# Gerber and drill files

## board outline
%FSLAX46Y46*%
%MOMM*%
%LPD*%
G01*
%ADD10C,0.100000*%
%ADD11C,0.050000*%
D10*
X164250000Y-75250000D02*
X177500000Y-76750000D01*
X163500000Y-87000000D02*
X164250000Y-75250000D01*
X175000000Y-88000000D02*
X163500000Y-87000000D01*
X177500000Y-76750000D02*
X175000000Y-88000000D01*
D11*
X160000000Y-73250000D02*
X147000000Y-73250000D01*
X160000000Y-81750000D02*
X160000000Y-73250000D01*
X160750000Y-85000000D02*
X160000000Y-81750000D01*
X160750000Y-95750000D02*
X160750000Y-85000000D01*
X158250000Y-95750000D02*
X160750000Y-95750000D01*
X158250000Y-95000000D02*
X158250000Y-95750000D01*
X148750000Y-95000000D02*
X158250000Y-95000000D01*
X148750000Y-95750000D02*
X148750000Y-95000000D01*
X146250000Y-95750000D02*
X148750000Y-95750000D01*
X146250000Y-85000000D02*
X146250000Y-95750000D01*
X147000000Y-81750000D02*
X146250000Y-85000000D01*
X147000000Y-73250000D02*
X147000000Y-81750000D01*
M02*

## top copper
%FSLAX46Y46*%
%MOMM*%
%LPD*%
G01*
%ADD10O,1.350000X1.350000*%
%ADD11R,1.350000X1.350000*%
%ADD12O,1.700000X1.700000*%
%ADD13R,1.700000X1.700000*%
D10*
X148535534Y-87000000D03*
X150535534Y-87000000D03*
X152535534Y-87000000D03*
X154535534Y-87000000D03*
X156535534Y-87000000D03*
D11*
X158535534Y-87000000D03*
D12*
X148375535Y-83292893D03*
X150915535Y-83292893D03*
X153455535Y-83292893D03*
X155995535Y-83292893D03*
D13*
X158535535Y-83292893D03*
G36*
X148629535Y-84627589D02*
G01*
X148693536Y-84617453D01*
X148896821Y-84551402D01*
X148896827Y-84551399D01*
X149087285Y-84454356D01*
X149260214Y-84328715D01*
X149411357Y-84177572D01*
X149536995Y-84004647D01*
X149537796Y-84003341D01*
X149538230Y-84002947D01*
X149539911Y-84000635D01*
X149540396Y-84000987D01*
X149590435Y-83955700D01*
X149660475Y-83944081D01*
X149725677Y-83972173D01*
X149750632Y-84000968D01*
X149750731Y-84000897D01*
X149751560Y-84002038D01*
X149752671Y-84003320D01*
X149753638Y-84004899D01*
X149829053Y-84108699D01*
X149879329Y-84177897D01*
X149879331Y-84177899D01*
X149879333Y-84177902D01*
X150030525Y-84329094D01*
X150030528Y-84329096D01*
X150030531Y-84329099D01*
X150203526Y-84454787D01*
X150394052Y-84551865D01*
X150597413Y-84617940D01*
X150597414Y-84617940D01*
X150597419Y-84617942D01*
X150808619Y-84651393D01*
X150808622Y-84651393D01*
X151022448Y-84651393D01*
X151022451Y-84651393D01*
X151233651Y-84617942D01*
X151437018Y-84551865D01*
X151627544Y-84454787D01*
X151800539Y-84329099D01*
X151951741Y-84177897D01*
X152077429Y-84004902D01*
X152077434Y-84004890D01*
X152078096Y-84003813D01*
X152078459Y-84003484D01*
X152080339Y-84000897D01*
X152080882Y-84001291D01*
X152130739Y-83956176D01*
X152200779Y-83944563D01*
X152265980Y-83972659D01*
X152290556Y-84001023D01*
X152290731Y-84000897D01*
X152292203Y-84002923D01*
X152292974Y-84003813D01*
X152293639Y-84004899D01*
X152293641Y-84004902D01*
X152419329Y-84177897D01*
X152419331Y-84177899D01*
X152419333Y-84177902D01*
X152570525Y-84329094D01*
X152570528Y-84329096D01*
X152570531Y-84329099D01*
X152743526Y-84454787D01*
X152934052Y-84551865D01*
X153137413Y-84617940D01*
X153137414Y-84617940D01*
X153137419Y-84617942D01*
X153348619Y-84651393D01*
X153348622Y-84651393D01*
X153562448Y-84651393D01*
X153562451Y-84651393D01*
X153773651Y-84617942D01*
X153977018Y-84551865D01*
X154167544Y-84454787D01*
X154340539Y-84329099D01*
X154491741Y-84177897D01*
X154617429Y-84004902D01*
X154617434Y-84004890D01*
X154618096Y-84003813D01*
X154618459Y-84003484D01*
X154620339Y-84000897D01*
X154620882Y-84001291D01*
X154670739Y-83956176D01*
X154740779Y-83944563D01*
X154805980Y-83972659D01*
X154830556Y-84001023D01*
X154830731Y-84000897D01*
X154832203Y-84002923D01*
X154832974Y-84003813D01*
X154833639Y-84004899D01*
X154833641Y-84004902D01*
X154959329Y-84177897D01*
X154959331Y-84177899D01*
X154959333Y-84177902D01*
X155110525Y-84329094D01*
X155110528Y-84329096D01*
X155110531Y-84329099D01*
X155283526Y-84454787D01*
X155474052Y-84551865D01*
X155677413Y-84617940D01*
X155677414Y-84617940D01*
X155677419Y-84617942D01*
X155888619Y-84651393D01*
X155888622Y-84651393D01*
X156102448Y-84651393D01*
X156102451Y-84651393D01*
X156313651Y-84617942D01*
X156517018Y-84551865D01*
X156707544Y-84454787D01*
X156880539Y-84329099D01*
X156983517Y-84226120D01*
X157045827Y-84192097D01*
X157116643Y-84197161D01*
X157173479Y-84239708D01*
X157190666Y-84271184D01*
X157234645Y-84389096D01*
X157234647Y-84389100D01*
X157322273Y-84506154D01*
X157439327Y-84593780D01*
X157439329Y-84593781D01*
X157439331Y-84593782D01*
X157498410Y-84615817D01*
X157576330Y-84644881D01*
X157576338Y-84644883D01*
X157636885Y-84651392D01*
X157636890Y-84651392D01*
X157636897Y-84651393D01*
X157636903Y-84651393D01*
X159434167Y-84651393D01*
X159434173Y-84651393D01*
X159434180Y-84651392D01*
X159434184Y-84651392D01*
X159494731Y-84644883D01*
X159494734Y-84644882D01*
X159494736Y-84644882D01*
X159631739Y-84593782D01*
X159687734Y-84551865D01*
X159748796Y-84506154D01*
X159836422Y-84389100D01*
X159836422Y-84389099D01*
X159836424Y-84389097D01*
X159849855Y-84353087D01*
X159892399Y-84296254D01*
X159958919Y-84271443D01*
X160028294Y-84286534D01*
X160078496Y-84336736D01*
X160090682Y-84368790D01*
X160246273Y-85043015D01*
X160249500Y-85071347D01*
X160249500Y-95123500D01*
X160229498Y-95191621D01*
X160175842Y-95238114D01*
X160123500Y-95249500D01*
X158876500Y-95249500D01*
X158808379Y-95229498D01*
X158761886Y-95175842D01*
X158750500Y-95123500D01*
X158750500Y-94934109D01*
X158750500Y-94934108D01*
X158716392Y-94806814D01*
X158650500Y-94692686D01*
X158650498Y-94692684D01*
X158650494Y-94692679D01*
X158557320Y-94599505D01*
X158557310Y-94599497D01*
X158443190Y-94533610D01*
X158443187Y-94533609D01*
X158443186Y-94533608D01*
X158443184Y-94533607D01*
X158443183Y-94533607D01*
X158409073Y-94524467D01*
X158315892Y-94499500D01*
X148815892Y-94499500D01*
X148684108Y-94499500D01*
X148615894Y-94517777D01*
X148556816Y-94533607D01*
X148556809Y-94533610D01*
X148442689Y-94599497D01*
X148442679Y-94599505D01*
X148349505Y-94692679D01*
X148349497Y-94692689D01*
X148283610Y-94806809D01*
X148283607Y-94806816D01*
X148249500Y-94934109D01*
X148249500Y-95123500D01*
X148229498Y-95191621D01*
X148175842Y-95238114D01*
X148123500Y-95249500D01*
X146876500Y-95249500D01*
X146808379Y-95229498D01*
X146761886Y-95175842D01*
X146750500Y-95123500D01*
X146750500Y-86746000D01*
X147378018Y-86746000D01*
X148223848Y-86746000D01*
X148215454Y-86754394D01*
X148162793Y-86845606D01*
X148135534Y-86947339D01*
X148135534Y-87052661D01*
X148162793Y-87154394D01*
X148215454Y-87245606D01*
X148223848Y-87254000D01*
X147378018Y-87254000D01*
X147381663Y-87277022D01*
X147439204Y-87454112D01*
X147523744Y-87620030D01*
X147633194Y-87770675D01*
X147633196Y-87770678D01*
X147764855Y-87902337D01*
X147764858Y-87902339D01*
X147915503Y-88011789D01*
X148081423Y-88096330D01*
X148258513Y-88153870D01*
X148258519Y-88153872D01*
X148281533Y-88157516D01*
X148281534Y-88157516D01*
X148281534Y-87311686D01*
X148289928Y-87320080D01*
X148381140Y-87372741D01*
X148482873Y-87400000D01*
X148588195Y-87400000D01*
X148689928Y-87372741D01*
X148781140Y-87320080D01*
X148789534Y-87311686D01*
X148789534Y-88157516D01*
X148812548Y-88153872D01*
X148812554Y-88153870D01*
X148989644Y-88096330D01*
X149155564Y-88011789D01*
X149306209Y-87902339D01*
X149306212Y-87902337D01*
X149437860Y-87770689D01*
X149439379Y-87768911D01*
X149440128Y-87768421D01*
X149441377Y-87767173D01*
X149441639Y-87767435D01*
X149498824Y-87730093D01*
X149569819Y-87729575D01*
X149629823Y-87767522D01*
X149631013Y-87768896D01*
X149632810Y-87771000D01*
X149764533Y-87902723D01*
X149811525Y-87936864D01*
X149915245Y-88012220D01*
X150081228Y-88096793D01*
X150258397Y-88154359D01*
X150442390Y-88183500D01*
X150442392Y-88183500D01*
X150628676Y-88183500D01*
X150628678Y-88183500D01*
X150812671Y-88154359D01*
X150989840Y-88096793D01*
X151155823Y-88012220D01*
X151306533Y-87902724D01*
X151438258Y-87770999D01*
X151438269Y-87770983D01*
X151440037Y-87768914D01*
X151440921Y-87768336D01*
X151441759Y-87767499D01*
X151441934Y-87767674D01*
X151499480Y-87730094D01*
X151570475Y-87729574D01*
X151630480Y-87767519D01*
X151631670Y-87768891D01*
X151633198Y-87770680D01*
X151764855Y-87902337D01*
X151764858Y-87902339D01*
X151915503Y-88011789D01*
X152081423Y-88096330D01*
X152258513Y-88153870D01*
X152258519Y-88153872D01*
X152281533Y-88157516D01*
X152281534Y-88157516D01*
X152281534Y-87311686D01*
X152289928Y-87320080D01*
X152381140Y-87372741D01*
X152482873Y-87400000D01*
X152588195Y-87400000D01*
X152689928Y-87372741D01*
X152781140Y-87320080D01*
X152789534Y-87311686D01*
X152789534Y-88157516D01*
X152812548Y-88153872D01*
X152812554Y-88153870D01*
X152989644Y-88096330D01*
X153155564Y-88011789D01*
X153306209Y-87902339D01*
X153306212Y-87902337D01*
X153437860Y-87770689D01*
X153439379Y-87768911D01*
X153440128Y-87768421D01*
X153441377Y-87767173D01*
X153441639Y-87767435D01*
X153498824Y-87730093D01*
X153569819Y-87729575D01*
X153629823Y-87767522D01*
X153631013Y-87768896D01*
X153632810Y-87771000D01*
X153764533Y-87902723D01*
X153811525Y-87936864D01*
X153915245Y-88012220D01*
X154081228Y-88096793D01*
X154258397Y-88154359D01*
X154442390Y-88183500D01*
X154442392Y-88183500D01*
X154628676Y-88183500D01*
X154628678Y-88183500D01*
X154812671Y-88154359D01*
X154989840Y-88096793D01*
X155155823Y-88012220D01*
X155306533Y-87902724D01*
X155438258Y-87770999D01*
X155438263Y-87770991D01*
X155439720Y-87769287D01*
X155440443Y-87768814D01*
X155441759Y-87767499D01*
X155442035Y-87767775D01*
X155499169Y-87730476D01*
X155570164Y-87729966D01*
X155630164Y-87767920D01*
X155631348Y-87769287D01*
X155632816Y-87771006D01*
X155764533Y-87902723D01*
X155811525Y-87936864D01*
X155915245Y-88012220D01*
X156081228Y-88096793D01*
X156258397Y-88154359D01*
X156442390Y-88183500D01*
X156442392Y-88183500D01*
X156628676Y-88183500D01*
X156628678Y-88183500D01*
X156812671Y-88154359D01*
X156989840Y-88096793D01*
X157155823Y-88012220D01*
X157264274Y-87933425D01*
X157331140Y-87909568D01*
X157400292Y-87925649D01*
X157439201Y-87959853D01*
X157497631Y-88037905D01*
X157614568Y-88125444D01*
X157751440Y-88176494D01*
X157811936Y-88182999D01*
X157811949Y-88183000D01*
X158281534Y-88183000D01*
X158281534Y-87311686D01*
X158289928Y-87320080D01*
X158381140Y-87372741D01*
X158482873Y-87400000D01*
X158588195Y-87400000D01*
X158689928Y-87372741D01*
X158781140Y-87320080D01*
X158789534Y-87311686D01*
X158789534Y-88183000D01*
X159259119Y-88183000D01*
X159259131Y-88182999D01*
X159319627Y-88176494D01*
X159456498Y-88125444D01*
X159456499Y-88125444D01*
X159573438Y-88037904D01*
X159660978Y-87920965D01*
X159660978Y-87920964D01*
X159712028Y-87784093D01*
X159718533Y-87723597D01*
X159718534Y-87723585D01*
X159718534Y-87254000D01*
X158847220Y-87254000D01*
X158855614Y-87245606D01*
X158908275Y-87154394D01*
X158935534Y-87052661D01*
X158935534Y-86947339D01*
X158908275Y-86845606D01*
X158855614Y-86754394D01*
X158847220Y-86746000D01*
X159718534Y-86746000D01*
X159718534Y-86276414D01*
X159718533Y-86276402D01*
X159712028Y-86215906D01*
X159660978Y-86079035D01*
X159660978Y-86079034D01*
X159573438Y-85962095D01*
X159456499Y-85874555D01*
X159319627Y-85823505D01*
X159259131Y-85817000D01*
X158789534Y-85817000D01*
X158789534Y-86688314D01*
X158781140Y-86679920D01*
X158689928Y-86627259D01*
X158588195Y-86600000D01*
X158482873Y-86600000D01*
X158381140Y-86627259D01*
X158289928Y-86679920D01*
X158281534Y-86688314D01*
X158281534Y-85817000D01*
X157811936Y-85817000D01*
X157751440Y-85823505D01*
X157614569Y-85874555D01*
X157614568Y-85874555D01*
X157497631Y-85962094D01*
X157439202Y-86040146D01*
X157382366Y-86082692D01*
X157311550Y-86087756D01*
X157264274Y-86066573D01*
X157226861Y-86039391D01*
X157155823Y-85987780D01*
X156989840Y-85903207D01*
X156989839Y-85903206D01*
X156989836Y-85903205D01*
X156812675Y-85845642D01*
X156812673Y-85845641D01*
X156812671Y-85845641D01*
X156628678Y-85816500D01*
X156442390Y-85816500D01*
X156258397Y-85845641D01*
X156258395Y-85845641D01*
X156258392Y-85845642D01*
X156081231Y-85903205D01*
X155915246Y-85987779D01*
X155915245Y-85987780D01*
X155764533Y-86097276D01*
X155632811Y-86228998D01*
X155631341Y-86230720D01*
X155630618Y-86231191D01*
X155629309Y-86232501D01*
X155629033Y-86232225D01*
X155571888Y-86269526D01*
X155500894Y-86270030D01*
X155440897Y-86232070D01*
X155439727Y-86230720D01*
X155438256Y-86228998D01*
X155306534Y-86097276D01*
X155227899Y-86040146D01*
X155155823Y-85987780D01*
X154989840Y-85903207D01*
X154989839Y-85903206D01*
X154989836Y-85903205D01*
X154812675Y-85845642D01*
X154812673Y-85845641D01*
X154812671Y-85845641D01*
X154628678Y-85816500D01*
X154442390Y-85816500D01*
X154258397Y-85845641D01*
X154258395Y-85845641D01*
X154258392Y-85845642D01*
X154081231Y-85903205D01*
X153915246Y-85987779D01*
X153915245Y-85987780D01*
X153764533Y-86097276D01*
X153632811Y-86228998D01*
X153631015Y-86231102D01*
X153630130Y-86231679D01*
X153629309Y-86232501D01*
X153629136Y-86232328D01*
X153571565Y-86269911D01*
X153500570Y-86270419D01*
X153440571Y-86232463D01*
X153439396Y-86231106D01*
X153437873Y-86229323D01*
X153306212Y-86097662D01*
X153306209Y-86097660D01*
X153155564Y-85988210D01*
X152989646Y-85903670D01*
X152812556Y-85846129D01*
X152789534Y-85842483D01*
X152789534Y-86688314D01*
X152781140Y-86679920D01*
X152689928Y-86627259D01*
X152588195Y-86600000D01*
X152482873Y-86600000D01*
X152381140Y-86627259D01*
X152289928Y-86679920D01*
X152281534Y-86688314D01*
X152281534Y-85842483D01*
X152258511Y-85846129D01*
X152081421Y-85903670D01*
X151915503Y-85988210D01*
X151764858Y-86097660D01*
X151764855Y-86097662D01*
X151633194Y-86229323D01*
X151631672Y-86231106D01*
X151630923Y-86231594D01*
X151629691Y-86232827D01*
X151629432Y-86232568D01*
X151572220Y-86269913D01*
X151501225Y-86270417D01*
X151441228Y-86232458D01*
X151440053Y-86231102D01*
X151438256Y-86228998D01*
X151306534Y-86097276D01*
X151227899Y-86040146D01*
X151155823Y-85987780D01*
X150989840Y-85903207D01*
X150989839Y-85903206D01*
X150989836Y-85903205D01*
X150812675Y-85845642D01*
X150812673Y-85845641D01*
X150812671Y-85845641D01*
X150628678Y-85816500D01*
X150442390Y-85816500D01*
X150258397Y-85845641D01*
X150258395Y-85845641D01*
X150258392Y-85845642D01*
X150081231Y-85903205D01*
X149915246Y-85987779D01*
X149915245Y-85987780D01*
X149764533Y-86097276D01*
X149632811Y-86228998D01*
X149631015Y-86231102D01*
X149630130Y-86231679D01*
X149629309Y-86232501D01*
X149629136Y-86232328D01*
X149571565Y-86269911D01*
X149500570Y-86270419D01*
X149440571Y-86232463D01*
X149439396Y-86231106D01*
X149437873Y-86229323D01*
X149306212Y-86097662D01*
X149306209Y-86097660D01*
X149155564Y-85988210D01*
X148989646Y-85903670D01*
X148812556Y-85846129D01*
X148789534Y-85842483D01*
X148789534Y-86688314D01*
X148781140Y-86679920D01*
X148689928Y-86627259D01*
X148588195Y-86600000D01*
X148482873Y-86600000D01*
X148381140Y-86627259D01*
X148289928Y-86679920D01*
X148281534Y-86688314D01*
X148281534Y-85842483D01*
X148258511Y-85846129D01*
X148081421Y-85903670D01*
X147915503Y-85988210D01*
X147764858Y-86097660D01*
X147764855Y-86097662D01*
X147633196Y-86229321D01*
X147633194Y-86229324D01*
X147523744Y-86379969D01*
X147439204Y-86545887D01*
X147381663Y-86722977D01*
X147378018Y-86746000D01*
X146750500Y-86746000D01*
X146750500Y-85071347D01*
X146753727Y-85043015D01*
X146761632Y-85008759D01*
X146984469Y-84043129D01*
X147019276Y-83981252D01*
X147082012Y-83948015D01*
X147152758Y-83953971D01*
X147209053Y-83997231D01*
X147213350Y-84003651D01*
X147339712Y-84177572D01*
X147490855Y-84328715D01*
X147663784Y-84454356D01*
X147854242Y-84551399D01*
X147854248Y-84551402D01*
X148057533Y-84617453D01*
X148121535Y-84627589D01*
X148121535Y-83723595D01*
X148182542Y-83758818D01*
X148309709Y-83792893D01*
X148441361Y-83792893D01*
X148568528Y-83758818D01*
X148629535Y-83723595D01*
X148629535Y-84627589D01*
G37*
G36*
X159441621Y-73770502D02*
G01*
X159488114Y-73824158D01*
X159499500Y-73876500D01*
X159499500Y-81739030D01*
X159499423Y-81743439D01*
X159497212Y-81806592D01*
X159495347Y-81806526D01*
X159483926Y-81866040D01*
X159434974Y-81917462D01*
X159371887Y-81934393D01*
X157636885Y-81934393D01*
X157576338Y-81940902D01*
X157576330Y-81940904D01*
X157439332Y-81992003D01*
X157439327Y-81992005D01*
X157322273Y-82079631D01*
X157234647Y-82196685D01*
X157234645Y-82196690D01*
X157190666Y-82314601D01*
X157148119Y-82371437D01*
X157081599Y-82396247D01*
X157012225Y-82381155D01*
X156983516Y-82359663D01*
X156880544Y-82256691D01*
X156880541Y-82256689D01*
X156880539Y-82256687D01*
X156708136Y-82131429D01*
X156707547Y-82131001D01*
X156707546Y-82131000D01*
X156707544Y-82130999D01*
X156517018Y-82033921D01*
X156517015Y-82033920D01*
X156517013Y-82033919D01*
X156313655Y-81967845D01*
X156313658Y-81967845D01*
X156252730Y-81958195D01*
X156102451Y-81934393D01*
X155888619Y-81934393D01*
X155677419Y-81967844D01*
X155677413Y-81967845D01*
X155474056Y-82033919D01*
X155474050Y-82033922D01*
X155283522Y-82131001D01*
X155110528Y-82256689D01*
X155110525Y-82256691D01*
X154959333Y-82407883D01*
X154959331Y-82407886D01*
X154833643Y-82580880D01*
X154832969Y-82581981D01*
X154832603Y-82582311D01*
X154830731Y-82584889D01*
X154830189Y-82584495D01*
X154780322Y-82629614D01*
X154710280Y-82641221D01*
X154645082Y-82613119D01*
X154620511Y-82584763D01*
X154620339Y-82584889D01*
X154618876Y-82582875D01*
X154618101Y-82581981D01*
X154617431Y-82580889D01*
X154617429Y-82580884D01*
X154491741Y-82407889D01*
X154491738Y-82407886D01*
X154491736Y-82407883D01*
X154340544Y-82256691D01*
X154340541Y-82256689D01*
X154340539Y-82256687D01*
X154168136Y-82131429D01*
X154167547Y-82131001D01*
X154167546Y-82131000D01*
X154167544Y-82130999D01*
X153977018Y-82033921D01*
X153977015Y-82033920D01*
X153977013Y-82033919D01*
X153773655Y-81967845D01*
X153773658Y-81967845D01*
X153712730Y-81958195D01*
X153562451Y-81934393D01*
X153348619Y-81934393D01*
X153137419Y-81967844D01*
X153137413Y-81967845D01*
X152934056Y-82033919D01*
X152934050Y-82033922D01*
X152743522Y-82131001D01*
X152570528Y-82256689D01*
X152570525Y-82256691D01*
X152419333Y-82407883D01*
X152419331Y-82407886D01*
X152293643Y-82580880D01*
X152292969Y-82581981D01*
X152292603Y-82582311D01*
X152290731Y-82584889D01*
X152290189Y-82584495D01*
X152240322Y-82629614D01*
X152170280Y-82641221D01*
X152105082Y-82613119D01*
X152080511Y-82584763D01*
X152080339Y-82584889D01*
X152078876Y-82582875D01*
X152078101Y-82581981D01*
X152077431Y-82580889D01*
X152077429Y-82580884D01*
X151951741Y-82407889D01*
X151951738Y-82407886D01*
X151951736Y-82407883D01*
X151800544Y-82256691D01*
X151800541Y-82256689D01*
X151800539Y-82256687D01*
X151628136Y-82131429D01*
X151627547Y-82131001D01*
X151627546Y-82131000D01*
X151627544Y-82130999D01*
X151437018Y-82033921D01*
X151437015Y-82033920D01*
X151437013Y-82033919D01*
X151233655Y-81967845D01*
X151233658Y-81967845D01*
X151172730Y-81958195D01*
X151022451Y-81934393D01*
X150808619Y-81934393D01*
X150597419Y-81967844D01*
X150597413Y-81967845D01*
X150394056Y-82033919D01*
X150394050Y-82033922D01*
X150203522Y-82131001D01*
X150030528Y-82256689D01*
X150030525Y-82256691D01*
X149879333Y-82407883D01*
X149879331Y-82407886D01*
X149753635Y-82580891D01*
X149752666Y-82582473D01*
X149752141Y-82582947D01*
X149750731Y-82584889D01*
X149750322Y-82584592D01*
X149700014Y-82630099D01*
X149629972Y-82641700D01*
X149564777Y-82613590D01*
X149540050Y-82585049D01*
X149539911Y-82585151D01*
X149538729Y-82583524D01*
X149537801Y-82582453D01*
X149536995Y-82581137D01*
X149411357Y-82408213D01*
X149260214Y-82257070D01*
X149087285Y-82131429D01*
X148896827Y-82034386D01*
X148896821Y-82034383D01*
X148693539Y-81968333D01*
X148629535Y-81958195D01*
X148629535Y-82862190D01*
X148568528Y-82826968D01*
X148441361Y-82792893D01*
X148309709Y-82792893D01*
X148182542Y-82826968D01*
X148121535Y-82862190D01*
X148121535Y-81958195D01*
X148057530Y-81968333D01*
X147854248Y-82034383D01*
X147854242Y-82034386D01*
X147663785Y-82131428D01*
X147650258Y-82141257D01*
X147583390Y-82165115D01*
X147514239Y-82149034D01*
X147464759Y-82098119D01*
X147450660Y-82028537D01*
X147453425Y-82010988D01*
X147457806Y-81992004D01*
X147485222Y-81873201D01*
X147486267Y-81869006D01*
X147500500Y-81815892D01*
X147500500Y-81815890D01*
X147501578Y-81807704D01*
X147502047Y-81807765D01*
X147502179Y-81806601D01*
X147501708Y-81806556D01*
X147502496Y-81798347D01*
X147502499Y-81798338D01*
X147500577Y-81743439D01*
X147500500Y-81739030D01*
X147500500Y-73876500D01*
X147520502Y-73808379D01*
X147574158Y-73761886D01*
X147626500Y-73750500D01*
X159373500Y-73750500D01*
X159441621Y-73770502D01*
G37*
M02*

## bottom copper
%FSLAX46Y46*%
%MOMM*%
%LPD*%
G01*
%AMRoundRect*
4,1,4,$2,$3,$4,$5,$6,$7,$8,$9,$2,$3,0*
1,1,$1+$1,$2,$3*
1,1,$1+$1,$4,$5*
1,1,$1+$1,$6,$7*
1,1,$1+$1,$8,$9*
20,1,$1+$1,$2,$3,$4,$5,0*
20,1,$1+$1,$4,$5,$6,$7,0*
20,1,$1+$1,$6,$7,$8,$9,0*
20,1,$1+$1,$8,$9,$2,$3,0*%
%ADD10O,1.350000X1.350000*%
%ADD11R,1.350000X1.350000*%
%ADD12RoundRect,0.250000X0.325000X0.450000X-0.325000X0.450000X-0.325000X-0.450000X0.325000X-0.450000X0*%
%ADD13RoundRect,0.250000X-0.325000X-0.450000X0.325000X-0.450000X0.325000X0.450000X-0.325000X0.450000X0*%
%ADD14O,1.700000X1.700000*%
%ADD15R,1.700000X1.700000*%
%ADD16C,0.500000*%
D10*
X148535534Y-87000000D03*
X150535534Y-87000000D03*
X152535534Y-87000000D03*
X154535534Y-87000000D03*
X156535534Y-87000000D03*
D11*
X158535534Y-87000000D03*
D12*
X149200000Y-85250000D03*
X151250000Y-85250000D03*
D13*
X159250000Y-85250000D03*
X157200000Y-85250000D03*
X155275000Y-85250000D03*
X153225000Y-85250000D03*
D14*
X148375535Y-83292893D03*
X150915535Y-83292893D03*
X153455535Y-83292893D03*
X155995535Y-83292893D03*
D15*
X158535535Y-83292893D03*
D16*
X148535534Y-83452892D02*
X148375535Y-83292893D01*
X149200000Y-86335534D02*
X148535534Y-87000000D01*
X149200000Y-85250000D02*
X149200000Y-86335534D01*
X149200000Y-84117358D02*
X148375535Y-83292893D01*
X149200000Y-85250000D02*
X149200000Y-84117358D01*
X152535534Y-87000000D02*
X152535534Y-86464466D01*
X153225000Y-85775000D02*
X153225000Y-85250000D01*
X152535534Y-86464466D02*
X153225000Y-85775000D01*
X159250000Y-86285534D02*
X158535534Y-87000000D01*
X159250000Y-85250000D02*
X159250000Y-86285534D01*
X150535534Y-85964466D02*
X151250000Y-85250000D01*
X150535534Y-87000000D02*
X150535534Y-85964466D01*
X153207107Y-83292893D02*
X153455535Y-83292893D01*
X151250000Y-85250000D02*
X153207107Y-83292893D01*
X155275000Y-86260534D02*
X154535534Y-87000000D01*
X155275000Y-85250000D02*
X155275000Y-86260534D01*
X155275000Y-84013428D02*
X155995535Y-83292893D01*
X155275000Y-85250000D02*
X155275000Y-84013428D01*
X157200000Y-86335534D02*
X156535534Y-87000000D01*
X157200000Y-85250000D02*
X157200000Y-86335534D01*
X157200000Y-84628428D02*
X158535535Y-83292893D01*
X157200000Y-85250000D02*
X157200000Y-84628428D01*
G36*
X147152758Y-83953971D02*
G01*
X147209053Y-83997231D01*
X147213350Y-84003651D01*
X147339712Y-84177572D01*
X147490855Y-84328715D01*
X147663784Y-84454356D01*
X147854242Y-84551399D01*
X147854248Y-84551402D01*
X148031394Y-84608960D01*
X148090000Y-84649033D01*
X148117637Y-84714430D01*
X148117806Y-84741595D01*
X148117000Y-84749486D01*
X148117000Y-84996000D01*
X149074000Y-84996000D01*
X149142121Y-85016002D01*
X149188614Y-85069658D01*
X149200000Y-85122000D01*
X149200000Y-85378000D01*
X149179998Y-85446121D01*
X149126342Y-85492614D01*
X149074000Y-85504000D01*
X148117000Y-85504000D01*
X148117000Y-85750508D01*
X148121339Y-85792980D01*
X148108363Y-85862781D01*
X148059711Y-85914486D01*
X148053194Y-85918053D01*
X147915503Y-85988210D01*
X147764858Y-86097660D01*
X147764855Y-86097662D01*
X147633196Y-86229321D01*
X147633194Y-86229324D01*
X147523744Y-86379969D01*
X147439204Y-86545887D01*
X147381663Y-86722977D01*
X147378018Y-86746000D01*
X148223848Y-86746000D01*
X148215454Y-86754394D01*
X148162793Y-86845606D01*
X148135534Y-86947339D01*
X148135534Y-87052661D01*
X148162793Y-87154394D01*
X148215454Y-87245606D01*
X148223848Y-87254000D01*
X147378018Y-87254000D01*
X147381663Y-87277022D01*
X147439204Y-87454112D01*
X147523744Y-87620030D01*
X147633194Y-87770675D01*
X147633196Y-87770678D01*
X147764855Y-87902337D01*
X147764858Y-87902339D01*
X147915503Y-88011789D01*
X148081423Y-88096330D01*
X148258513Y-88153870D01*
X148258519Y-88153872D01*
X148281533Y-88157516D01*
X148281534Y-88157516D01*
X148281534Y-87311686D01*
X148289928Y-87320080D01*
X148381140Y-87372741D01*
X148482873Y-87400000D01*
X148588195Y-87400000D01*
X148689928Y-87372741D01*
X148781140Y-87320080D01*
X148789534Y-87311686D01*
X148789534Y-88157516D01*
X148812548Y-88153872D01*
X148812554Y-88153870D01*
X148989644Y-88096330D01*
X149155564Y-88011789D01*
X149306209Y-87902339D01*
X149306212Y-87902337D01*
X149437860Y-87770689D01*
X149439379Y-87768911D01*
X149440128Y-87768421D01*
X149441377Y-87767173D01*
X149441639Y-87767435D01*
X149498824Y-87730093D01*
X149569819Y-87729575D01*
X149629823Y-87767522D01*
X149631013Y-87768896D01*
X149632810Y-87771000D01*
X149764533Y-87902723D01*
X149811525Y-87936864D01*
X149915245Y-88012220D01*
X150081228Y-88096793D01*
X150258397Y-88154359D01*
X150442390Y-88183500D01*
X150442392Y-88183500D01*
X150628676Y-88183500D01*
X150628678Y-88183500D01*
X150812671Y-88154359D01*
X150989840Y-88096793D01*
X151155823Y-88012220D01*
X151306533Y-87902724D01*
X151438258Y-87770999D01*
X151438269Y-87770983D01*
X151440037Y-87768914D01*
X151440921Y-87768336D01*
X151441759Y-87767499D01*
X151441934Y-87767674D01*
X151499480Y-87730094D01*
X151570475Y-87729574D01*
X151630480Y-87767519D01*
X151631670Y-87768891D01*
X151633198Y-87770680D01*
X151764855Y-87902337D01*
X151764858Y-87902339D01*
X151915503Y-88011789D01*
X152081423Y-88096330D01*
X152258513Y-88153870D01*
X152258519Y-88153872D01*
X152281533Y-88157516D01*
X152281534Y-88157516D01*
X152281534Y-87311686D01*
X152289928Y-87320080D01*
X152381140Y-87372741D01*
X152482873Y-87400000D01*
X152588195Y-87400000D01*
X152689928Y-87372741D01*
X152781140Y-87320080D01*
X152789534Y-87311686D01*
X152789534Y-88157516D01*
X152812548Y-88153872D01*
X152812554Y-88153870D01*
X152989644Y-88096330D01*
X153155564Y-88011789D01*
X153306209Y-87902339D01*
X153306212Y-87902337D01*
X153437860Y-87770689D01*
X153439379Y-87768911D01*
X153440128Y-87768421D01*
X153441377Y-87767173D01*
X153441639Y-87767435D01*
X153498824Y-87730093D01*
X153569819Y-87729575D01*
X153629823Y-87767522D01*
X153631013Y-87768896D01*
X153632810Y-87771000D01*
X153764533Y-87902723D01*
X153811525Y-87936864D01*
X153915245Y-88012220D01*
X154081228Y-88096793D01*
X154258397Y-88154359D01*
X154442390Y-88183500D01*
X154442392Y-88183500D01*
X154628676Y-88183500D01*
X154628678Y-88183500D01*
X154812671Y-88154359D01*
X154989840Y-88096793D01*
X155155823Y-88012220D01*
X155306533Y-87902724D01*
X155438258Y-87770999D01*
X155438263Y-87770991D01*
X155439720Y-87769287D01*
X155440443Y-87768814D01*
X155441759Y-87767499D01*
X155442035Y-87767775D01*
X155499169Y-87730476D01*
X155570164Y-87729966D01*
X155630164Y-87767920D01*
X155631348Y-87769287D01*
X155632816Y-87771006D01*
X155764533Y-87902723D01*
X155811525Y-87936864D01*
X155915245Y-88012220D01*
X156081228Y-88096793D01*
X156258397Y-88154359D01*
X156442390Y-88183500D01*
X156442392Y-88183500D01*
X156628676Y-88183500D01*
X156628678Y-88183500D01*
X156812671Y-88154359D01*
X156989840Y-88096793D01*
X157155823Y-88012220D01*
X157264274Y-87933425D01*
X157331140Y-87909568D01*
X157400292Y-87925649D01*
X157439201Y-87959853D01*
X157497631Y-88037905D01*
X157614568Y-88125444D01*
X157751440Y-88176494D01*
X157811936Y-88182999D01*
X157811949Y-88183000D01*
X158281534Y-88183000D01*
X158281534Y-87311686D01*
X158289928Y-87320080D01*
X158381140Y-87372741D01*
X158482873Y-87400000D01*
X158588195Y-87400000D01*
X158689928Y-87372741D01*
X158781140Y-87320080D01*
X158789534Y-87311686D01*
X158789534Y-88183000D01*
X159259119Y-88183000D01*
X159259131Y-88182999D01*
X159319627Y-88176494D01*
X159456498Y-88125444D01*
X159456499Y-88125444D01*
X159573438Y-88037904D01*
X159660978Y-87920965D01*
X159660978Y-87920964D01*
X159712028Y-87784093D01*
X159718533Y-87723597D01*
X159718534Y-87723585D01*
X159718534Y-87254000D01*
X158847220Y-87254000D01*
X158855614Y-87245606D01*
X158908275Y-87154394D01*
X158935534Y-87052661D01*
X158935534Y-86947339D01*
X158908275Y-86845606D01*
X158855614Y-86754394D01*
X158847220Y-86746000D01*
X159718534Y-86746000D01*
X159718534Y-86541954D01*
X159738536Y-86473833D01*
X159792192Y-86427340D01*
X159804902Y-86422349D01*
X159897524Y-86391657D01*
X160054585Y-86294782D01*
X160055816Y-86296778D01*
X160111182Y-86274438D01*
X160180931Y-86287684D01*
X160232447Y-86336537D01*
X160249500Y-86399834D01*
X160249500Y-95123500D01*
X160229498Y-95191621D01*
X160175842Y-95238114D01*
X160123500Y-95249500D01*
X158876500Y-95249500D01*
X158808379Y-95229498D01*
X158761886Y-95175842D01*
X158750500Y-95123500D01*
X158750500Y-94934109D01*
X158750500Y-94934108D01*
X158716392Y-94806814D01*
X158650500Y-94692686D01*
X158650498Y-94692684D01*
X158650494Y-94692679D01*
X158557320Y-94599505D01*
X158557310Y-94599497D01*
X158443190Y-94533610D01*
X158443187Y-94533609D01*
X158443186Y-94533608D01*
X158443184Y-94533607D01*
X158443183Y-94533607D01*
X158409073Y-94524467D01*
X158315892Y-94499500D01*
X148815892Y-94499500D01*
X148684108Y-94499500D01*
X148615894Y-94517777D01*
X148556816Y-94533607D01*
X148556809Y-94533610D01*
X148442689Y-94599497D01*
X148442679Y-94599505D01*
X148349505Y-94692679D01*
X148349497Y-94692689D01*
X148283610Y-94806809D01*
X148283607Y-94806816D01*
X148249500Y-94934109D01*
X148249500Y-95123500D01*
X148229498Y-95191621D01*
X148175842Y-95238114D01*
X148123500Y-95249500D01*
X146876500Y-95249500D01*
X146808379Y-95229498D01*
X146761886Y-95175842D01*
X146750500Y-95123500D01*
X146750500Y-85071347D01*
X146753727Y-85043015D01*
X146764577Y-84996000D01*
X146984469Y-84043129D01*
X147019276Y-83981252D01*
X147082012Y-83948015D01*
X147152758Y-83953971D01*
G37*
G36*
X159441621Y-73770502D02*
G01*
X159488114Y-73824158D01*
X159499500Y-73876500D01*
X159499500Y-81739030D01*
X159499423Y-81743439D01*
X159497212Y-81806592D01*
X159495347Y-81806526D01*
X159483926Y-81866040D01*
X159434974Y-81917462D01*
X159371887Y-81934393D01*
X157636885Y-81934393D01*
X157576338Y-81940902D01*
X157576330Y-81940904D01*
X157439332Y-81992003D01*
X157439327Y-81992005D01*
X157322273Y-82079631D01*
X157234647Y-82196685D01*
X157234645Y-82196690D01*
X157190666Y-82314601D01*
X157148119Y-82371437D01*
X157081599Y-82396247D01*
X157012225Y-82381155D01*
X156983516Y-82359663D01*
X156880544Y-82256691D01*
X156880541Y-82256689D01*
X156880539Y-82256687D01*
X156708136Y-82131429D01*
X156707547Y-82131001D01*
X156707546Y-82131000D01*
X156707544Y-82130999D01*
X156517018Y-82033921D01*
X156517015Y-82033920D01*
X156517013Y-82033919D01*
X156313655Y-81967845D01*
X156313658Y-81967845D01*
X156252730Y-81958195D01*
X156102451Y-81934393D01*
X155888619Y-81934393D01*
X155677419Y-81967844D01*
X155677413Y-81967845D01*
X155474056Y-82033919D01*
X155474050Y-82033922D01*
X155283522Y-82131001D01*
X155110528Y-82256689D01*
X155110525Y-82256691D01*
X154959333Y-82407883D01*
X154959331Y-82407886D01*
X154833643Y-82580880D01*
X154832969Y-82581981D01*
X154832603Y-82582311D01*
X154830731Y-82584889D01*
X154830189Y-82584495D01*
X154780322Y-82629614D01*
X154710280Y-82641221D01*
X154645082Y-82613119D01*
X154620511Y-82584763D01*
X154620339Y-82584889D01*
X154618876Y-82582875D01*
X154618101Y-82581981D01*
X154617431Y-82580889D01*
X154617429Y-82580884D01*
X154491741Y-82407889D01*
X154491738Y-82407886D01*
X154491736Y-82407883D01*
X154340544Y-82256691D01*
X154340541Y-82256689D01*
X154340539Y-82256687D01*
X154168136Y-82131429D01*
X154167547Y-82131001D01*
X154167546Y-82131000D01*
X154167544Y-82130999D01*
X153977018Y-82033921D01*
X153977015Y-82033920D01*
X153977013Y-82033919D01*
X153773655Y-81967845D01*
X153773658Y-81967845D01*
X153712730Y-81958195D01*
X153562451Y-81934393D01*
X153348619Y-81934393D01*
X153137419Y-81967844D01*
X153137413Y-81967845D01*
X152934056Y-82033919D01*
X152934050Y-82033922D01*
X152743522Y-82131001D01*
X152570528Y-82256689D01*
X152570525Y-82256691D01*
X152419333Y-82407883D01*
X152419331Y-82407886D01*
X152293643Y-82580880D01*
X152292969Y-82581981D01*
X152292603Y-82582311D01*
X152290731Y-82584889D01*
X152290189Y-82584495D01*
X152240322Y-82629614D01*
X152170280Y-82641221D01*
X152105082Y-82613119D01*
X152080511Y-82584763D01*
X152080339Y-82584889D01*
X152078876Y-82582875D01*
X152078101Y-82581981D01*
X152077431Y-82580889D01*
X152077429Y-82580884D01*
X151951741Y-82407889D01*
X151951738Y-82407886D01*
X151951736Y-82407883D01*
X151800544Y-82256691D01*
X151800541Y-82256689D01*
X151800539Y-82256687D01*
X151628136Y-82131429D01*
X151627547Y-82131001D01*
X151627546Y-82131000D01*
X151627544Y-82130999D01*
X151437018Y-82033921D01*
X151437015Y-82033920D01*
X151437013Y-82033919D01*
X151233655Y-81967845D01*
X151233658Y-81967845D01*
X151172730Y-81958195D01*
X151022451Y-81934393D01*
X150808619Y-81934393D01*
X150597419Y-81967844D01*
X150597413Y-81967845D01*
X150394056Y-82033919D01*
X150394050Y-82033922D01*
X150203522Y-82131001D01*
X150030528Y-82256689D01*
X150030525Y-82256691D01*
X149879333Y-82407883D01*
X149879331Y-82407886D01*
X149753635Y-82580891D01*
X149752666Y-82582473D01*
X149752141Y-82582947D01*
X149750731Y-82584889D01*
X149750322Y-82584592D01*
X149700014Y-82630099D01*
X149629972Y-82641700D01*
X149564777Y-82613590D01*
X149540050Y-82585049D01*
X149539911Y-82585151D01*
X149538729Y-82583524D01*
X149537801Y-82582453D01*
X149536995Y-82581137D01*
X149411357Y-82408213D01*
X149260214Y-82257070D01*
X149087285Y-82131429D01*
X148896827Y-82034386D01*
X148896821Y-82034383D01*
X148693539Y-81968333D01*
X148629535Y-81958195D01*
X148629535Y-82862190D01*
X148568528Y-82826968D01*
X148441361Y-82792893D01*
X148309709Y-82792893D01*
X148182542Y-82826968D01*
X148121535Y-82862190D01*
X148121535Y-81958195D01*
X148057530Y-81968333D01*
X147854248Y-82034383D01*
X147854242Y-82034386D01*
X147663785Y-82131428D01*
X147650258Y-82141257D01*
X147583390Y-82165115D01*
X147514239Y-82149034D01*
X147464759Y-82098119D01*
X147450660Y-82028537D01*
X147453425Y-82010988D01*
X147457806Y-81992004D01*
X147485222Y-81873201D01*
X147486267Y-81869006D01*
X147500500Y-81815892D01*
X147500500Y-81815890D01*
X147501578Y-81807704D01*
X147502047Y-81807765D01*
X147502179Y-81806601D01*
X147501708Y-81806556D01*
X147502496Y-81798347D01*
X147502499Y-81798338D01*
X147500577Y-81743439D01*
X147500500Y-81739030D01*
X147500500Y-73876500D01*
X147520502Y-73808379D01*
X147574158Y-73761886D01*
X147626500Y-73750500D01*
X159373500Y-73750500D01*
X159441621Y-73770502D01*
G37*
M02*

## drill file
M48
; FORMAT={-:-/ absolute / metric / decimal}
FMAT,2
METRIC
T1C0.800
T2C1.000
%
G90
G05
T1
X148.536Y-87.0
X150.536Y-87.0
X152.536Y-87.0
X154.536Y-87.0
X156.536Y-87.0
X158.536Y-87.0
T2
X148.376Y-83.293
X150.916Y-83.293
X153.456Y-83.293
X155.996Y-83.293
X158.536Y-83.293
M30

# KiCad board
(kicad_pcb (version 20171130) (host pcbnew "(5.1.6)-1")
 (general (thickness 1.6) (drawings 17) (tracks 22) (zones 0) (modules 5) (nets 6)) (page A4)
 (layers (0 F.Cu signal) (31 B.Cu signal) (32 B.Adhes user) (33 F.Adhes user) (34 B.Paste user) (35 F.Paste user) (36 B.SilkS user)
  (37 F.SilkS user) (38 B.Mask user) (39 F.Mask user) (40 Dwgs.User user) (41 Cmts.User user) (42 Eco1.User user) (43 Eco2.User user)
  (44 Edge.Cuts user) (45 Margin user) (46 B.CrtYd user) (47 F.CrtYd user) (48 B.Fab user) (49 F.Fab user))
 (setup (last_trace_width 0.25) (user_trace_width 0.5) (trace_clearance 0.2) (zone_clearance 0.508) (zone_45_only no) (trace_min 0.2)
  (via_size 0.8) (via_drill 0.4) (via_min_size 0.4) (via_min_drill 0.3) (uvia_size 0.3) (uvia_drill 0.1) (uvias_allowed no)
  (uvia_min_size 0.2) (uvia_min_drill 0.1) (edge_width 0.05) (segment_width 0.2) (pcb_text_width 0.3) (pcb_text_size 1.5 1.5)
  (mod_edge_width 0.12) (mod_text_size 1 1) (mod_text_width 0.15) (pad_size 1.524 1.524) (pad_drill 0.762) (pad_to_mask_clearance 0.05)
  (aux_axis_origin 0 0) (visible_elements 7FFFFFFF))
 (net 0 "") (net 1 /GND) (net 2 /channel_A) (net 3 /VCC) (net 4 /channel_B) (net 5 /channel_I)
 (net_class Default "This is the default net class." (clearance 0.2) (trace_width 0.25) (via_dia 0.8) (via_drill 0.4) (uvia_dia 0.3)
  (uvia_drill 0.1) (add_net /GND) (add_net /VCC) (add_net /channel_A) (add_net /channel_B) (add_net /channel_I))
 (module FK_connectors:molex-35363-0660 (layer F.Cu) (at 158.535534 87 270)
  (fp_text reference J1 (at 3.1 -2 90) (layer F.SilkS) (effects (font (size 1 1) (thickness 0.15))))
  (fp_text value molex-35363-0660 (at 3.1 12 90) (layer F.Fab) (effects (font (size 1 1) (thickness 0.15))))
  (pad 6 thru_hole oval (at 0 10 270) (size 1.35 1.35) (drill 0.8) (layers *.Cu *.Mask) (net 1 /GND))
  (pad 5 thru_hole oval (at 0 8 270) (size 1.35 1.35) (drill 0.8) (layers *.Cu *.Mask) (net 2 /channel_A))
  (pad 4 thru_hole oval (at 0 6 270) (size 1.35 1.35) (drill 0.8) (layers *.Cu *.Mask) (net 1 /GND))
  (pad 3 thru_hole oval (at 0 4 270) (size 1.35 1.35) (drill 0.8) (layers *.Cu *.Mask) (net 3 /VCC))
  (pad 2 thru_hole oval (at 0 2 270) (size 1.35 1.35) (drill 0.8) (layers *.Cu *.Mask) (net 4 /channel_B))
  (pad 1 thru_hole rect (at 0 0 270) (size 1.35 1.35) (drill 0.8) (layers *.Cu *.Mask) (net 1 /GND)))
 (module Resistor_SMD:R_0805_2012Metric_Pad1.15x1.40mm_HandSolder (layer B.Cu) (at 150.225 85.25 180)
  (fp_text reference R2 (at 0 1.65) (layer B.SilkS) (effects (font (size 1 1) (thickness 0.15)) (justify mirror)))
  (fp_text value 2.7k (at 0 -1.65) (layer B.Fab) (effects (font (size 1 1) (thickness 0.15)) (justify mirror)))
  (pad 2 smd roundrect (at 1.025 0 180) (size 1.15 1.4) (layers B.Cu B.Paste B.Mask) (roundrect_rratio 0.217391) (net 1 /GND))
  (pad 1 smd roundrect (at -1.025 0 180) (size 1.15 1.4) (layers B.Cu B.Paste B.Mask) (roundrect_rratio 0.217391) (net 2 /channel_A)))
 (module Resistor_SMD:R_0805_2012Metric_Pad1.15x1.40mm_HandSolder (layer B.Cu) (at 158.225 85.25)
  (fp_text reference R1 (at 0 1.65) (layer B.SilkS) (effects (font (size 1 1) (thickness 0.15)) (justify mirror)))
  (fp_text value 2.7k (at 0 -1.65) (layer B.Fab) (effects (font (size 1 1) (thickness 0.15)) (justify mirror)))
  (pad 2 smd roundrect (at 1.025 0) (size 1.15 1.4) (layers B.Cu B.Paste B.Mask) (roundrect_rratio 0.217391) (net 1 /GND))
  (pad 1 smd roundrect (at -1.025 0) (size 1.15 1.4) (layers B.Cu B.Paste B.Mask) (roundrect_rratio 0.217391) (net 4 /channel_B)))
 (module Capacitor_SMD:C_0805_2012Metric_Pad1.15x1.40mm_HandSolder (layer B.Cu) (at 154.25 85.25)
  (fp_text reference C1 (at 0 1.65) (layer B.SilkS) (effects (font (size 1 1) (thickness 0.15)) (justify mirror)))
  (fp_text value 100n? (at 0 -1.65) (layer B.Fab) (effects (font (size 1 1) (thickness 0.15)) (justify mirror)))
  (pad 2 smd roundrect (at 1.025 0) (size 1.15 1.4) (layers B.Cu B.Paste B.Mask) (roundrect_rratio 0.217391) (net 3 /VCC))
  (pad 1 smd roundrect (at -1.025 0) (size 1.15 1.4) (layers B.Cu B.Paste B.Mask) (roundrect_rratio 0.217391) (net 1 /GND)))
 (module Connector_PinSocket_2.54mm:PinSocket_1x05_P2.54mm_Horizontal (layer F.Cu) (at 158.535535 83.292893 270)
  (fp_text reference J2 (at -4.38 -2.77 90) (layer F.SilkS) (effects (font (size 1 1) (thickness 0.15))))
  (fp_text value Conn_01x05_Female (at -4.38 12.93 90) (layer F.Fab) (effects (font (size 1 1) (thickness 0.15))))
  (pad 5 thru_hole oval (at 0 10.16 270) (size 1.7 1.7) (drill 1) (layers *.Cu *.Mask) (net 1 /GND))
  (pad 4 thru_hole oval (at 0 7.62 270) (size 1.7 1.7) (drill 1) (layers *.Cu *.Mask) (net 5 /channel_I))
  (pad 3 thru_hole oval (at 0 5.08 270) (size 1.7 1.7) (drill 1) (layers *.Cu *.Mask) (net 2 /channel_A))
  (pad 2 thru_hole oval (at 0 2.54 270) (size 1.7 1.7) (drill 1) (layers *.Cu *.Mask) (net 3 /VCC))
  (pad 1 thru_hole rect (at 0 0 270) (size 1.7 1.7) (drill 1) (layers *.Cu *.Mask) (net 4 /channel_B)))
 (gr_line (start 164.25 75.25) (end 177.5 76.75) (layer Edge.Cuts) (width 0.1))
 (gr_line (start 163.5 87) (end 164.25 75.25) (layer Edge.Cuts) (width 0.1))
 (gr_line (start 175 88) (end 163.5 87) (layer Edge.Cuts) (width 0.1))
 (gr_line (start 177.5 76.75) (end 175 88) (layer Edge.Cuts) (width 0.1))
 (gr_line (start 160 73.25) (end 147 73.25) (layer Edge.Cuts) (width 0.05))
 (gr_line (start 160 81.75) (end 160 73.25) (layer Edge.Cuts) (width 0.05))
 (gr_line (start 160.75 85) (end 160 81.75) (layer Edge.Cuts) (width 0.05))
 (gr_line (start 160.75 95.75) (end 160.75 85) (layer Edge.Cuts) (width 0.05))
 (gr_line (start 158.25 95.75) (end 160.75 95.75) (layer Edge.Cuts) (width 0.05))
 (gr_line (start 158.25 95) (end 158.25 95.75) (layer Edge.Cuts) (width 0.05))
 (gr_line (start 148.75 95) (end 158.25 95) (layer Edge.Cuts) (width 0.05))
 (gr_line (start 148.75 95.75) (end 148.75 95) (layer Edge.Cuts) (width 0.05))
 (gr_line (start 146.25 95.75) (end 148.75 95.75) (layer Edge.Cuts) (width 0.05))
 (gr_line (start 146.25 85) (end 146.25 95.75) (layer Edge.Cuts) (width 0.05))
 (gr_line (start 147 81.75) (end 146.25 85) (layer Edge.Cuts) (width 0.05))
 (gr_line (start 147 73.25) (end 147 81.75) (layer Edge.Cuts) (width 0.05))
 (segment (start 148.535534 83.452892) (end 148.375535 83.292893) (width 0.5) (layer B.Cu) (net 1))
 (segment (start 149.2 86.335534) (end 148.535534 87) (width 0.5) (layer B.Cu) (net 1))
 (segment (start 149.2 85.25) (end 149.2 86.335534) (width 0.5) (layer B.Cu) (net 1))
 (segment (start 149.2 84.117358) (end 148.375535 83.292893) (width 0.5) (layer B.Cu) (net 1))
 (segment (start 149.2 85.25) (end 149.2 84.117358) (width 0.5) (layer B.Cu) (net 1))
 (segment (start 152.535534 87) (end 152.535534 86.464466) (width 0.5) (layer B.Cu) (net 1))
 (segment (start 153.225 85.775) (end 153.225 85.25) (width 0.5) (layer B.Cu) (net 1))
 (segment (start 152.535534 86.464466) (end 153.225 85.775) (width 0.5) (layer B.Cu) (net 1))
 (segment (start 159.25 86.285534) (end 158.535534 87) (width 0.5) (layer B.Cu) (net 1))
 (segment (start 159.25 85.25) (end 159.25 86.285534) (width 0.5) (layer B.Cu) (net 1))
 (segment (start 150.535534 85.964466) (end 151.25 85.25) (width 0.5) (layer B.Cu) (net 2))
 (segment (start 150.535534 87) (end 150.535534 85.964466) (width 0.5) (layer B.Cu) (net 2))
 (segment (start 153.207107 83.292893) (end 153.455535 83.292893) (width 0.5) (layer B.Cu) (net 2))
 (segment (start 151.25 85.25) (end 153.207107 83.292893) (width 0.5) (layer B.Cu) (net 2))
 (segment (start 155.275 86.260534) (end 154.535534 87) (width 0.5) (layer B.Cu) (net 3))
 (segment (start 155.275 85.25) (end 155.275 86.260534) (width 0.5) (layer B.Cu) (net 3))
 (segment (start 155.275 84.013428) (end 155.995535 83.292893) (width 0.5) (layer B.Cu) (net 3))
 (segment (start 155.275 85.25) (end 155.275 84.013428) (width 0.5) (layer B.Cu) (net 3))
 (segment (start 157.2 86.335534) (end 156.535534 87) (width 0.5) (layer B.Cu) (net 4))
 (segment (start 157.2 85.25) (end 157.2 86.335534) (width 0.5) (layer B.Cu) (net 4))
 (segment (start 157.2 84.628428) (end 158.535535 83.292893) (width 0.5) (layer B.Cu) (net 4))
 (segment (start 157.2 85.25) (end 157.2 84.628428) (width 0.5) (layer B.Cu) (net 4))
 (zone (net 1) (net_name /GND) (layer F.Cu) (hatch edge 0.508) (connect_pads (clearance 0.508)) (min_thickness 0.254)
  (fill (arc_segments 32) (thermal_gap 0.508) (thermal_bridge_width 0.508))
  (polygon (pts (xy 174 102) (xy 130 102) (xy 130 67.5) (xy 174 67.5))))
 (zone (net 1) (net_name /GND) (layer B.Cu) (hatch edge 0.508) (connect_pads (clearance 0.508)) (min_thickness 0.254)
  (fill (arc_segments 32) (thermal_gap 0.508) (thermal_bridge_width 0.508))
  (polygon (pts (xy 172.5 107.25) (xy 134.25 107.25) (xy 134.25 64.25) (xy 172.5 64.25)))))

